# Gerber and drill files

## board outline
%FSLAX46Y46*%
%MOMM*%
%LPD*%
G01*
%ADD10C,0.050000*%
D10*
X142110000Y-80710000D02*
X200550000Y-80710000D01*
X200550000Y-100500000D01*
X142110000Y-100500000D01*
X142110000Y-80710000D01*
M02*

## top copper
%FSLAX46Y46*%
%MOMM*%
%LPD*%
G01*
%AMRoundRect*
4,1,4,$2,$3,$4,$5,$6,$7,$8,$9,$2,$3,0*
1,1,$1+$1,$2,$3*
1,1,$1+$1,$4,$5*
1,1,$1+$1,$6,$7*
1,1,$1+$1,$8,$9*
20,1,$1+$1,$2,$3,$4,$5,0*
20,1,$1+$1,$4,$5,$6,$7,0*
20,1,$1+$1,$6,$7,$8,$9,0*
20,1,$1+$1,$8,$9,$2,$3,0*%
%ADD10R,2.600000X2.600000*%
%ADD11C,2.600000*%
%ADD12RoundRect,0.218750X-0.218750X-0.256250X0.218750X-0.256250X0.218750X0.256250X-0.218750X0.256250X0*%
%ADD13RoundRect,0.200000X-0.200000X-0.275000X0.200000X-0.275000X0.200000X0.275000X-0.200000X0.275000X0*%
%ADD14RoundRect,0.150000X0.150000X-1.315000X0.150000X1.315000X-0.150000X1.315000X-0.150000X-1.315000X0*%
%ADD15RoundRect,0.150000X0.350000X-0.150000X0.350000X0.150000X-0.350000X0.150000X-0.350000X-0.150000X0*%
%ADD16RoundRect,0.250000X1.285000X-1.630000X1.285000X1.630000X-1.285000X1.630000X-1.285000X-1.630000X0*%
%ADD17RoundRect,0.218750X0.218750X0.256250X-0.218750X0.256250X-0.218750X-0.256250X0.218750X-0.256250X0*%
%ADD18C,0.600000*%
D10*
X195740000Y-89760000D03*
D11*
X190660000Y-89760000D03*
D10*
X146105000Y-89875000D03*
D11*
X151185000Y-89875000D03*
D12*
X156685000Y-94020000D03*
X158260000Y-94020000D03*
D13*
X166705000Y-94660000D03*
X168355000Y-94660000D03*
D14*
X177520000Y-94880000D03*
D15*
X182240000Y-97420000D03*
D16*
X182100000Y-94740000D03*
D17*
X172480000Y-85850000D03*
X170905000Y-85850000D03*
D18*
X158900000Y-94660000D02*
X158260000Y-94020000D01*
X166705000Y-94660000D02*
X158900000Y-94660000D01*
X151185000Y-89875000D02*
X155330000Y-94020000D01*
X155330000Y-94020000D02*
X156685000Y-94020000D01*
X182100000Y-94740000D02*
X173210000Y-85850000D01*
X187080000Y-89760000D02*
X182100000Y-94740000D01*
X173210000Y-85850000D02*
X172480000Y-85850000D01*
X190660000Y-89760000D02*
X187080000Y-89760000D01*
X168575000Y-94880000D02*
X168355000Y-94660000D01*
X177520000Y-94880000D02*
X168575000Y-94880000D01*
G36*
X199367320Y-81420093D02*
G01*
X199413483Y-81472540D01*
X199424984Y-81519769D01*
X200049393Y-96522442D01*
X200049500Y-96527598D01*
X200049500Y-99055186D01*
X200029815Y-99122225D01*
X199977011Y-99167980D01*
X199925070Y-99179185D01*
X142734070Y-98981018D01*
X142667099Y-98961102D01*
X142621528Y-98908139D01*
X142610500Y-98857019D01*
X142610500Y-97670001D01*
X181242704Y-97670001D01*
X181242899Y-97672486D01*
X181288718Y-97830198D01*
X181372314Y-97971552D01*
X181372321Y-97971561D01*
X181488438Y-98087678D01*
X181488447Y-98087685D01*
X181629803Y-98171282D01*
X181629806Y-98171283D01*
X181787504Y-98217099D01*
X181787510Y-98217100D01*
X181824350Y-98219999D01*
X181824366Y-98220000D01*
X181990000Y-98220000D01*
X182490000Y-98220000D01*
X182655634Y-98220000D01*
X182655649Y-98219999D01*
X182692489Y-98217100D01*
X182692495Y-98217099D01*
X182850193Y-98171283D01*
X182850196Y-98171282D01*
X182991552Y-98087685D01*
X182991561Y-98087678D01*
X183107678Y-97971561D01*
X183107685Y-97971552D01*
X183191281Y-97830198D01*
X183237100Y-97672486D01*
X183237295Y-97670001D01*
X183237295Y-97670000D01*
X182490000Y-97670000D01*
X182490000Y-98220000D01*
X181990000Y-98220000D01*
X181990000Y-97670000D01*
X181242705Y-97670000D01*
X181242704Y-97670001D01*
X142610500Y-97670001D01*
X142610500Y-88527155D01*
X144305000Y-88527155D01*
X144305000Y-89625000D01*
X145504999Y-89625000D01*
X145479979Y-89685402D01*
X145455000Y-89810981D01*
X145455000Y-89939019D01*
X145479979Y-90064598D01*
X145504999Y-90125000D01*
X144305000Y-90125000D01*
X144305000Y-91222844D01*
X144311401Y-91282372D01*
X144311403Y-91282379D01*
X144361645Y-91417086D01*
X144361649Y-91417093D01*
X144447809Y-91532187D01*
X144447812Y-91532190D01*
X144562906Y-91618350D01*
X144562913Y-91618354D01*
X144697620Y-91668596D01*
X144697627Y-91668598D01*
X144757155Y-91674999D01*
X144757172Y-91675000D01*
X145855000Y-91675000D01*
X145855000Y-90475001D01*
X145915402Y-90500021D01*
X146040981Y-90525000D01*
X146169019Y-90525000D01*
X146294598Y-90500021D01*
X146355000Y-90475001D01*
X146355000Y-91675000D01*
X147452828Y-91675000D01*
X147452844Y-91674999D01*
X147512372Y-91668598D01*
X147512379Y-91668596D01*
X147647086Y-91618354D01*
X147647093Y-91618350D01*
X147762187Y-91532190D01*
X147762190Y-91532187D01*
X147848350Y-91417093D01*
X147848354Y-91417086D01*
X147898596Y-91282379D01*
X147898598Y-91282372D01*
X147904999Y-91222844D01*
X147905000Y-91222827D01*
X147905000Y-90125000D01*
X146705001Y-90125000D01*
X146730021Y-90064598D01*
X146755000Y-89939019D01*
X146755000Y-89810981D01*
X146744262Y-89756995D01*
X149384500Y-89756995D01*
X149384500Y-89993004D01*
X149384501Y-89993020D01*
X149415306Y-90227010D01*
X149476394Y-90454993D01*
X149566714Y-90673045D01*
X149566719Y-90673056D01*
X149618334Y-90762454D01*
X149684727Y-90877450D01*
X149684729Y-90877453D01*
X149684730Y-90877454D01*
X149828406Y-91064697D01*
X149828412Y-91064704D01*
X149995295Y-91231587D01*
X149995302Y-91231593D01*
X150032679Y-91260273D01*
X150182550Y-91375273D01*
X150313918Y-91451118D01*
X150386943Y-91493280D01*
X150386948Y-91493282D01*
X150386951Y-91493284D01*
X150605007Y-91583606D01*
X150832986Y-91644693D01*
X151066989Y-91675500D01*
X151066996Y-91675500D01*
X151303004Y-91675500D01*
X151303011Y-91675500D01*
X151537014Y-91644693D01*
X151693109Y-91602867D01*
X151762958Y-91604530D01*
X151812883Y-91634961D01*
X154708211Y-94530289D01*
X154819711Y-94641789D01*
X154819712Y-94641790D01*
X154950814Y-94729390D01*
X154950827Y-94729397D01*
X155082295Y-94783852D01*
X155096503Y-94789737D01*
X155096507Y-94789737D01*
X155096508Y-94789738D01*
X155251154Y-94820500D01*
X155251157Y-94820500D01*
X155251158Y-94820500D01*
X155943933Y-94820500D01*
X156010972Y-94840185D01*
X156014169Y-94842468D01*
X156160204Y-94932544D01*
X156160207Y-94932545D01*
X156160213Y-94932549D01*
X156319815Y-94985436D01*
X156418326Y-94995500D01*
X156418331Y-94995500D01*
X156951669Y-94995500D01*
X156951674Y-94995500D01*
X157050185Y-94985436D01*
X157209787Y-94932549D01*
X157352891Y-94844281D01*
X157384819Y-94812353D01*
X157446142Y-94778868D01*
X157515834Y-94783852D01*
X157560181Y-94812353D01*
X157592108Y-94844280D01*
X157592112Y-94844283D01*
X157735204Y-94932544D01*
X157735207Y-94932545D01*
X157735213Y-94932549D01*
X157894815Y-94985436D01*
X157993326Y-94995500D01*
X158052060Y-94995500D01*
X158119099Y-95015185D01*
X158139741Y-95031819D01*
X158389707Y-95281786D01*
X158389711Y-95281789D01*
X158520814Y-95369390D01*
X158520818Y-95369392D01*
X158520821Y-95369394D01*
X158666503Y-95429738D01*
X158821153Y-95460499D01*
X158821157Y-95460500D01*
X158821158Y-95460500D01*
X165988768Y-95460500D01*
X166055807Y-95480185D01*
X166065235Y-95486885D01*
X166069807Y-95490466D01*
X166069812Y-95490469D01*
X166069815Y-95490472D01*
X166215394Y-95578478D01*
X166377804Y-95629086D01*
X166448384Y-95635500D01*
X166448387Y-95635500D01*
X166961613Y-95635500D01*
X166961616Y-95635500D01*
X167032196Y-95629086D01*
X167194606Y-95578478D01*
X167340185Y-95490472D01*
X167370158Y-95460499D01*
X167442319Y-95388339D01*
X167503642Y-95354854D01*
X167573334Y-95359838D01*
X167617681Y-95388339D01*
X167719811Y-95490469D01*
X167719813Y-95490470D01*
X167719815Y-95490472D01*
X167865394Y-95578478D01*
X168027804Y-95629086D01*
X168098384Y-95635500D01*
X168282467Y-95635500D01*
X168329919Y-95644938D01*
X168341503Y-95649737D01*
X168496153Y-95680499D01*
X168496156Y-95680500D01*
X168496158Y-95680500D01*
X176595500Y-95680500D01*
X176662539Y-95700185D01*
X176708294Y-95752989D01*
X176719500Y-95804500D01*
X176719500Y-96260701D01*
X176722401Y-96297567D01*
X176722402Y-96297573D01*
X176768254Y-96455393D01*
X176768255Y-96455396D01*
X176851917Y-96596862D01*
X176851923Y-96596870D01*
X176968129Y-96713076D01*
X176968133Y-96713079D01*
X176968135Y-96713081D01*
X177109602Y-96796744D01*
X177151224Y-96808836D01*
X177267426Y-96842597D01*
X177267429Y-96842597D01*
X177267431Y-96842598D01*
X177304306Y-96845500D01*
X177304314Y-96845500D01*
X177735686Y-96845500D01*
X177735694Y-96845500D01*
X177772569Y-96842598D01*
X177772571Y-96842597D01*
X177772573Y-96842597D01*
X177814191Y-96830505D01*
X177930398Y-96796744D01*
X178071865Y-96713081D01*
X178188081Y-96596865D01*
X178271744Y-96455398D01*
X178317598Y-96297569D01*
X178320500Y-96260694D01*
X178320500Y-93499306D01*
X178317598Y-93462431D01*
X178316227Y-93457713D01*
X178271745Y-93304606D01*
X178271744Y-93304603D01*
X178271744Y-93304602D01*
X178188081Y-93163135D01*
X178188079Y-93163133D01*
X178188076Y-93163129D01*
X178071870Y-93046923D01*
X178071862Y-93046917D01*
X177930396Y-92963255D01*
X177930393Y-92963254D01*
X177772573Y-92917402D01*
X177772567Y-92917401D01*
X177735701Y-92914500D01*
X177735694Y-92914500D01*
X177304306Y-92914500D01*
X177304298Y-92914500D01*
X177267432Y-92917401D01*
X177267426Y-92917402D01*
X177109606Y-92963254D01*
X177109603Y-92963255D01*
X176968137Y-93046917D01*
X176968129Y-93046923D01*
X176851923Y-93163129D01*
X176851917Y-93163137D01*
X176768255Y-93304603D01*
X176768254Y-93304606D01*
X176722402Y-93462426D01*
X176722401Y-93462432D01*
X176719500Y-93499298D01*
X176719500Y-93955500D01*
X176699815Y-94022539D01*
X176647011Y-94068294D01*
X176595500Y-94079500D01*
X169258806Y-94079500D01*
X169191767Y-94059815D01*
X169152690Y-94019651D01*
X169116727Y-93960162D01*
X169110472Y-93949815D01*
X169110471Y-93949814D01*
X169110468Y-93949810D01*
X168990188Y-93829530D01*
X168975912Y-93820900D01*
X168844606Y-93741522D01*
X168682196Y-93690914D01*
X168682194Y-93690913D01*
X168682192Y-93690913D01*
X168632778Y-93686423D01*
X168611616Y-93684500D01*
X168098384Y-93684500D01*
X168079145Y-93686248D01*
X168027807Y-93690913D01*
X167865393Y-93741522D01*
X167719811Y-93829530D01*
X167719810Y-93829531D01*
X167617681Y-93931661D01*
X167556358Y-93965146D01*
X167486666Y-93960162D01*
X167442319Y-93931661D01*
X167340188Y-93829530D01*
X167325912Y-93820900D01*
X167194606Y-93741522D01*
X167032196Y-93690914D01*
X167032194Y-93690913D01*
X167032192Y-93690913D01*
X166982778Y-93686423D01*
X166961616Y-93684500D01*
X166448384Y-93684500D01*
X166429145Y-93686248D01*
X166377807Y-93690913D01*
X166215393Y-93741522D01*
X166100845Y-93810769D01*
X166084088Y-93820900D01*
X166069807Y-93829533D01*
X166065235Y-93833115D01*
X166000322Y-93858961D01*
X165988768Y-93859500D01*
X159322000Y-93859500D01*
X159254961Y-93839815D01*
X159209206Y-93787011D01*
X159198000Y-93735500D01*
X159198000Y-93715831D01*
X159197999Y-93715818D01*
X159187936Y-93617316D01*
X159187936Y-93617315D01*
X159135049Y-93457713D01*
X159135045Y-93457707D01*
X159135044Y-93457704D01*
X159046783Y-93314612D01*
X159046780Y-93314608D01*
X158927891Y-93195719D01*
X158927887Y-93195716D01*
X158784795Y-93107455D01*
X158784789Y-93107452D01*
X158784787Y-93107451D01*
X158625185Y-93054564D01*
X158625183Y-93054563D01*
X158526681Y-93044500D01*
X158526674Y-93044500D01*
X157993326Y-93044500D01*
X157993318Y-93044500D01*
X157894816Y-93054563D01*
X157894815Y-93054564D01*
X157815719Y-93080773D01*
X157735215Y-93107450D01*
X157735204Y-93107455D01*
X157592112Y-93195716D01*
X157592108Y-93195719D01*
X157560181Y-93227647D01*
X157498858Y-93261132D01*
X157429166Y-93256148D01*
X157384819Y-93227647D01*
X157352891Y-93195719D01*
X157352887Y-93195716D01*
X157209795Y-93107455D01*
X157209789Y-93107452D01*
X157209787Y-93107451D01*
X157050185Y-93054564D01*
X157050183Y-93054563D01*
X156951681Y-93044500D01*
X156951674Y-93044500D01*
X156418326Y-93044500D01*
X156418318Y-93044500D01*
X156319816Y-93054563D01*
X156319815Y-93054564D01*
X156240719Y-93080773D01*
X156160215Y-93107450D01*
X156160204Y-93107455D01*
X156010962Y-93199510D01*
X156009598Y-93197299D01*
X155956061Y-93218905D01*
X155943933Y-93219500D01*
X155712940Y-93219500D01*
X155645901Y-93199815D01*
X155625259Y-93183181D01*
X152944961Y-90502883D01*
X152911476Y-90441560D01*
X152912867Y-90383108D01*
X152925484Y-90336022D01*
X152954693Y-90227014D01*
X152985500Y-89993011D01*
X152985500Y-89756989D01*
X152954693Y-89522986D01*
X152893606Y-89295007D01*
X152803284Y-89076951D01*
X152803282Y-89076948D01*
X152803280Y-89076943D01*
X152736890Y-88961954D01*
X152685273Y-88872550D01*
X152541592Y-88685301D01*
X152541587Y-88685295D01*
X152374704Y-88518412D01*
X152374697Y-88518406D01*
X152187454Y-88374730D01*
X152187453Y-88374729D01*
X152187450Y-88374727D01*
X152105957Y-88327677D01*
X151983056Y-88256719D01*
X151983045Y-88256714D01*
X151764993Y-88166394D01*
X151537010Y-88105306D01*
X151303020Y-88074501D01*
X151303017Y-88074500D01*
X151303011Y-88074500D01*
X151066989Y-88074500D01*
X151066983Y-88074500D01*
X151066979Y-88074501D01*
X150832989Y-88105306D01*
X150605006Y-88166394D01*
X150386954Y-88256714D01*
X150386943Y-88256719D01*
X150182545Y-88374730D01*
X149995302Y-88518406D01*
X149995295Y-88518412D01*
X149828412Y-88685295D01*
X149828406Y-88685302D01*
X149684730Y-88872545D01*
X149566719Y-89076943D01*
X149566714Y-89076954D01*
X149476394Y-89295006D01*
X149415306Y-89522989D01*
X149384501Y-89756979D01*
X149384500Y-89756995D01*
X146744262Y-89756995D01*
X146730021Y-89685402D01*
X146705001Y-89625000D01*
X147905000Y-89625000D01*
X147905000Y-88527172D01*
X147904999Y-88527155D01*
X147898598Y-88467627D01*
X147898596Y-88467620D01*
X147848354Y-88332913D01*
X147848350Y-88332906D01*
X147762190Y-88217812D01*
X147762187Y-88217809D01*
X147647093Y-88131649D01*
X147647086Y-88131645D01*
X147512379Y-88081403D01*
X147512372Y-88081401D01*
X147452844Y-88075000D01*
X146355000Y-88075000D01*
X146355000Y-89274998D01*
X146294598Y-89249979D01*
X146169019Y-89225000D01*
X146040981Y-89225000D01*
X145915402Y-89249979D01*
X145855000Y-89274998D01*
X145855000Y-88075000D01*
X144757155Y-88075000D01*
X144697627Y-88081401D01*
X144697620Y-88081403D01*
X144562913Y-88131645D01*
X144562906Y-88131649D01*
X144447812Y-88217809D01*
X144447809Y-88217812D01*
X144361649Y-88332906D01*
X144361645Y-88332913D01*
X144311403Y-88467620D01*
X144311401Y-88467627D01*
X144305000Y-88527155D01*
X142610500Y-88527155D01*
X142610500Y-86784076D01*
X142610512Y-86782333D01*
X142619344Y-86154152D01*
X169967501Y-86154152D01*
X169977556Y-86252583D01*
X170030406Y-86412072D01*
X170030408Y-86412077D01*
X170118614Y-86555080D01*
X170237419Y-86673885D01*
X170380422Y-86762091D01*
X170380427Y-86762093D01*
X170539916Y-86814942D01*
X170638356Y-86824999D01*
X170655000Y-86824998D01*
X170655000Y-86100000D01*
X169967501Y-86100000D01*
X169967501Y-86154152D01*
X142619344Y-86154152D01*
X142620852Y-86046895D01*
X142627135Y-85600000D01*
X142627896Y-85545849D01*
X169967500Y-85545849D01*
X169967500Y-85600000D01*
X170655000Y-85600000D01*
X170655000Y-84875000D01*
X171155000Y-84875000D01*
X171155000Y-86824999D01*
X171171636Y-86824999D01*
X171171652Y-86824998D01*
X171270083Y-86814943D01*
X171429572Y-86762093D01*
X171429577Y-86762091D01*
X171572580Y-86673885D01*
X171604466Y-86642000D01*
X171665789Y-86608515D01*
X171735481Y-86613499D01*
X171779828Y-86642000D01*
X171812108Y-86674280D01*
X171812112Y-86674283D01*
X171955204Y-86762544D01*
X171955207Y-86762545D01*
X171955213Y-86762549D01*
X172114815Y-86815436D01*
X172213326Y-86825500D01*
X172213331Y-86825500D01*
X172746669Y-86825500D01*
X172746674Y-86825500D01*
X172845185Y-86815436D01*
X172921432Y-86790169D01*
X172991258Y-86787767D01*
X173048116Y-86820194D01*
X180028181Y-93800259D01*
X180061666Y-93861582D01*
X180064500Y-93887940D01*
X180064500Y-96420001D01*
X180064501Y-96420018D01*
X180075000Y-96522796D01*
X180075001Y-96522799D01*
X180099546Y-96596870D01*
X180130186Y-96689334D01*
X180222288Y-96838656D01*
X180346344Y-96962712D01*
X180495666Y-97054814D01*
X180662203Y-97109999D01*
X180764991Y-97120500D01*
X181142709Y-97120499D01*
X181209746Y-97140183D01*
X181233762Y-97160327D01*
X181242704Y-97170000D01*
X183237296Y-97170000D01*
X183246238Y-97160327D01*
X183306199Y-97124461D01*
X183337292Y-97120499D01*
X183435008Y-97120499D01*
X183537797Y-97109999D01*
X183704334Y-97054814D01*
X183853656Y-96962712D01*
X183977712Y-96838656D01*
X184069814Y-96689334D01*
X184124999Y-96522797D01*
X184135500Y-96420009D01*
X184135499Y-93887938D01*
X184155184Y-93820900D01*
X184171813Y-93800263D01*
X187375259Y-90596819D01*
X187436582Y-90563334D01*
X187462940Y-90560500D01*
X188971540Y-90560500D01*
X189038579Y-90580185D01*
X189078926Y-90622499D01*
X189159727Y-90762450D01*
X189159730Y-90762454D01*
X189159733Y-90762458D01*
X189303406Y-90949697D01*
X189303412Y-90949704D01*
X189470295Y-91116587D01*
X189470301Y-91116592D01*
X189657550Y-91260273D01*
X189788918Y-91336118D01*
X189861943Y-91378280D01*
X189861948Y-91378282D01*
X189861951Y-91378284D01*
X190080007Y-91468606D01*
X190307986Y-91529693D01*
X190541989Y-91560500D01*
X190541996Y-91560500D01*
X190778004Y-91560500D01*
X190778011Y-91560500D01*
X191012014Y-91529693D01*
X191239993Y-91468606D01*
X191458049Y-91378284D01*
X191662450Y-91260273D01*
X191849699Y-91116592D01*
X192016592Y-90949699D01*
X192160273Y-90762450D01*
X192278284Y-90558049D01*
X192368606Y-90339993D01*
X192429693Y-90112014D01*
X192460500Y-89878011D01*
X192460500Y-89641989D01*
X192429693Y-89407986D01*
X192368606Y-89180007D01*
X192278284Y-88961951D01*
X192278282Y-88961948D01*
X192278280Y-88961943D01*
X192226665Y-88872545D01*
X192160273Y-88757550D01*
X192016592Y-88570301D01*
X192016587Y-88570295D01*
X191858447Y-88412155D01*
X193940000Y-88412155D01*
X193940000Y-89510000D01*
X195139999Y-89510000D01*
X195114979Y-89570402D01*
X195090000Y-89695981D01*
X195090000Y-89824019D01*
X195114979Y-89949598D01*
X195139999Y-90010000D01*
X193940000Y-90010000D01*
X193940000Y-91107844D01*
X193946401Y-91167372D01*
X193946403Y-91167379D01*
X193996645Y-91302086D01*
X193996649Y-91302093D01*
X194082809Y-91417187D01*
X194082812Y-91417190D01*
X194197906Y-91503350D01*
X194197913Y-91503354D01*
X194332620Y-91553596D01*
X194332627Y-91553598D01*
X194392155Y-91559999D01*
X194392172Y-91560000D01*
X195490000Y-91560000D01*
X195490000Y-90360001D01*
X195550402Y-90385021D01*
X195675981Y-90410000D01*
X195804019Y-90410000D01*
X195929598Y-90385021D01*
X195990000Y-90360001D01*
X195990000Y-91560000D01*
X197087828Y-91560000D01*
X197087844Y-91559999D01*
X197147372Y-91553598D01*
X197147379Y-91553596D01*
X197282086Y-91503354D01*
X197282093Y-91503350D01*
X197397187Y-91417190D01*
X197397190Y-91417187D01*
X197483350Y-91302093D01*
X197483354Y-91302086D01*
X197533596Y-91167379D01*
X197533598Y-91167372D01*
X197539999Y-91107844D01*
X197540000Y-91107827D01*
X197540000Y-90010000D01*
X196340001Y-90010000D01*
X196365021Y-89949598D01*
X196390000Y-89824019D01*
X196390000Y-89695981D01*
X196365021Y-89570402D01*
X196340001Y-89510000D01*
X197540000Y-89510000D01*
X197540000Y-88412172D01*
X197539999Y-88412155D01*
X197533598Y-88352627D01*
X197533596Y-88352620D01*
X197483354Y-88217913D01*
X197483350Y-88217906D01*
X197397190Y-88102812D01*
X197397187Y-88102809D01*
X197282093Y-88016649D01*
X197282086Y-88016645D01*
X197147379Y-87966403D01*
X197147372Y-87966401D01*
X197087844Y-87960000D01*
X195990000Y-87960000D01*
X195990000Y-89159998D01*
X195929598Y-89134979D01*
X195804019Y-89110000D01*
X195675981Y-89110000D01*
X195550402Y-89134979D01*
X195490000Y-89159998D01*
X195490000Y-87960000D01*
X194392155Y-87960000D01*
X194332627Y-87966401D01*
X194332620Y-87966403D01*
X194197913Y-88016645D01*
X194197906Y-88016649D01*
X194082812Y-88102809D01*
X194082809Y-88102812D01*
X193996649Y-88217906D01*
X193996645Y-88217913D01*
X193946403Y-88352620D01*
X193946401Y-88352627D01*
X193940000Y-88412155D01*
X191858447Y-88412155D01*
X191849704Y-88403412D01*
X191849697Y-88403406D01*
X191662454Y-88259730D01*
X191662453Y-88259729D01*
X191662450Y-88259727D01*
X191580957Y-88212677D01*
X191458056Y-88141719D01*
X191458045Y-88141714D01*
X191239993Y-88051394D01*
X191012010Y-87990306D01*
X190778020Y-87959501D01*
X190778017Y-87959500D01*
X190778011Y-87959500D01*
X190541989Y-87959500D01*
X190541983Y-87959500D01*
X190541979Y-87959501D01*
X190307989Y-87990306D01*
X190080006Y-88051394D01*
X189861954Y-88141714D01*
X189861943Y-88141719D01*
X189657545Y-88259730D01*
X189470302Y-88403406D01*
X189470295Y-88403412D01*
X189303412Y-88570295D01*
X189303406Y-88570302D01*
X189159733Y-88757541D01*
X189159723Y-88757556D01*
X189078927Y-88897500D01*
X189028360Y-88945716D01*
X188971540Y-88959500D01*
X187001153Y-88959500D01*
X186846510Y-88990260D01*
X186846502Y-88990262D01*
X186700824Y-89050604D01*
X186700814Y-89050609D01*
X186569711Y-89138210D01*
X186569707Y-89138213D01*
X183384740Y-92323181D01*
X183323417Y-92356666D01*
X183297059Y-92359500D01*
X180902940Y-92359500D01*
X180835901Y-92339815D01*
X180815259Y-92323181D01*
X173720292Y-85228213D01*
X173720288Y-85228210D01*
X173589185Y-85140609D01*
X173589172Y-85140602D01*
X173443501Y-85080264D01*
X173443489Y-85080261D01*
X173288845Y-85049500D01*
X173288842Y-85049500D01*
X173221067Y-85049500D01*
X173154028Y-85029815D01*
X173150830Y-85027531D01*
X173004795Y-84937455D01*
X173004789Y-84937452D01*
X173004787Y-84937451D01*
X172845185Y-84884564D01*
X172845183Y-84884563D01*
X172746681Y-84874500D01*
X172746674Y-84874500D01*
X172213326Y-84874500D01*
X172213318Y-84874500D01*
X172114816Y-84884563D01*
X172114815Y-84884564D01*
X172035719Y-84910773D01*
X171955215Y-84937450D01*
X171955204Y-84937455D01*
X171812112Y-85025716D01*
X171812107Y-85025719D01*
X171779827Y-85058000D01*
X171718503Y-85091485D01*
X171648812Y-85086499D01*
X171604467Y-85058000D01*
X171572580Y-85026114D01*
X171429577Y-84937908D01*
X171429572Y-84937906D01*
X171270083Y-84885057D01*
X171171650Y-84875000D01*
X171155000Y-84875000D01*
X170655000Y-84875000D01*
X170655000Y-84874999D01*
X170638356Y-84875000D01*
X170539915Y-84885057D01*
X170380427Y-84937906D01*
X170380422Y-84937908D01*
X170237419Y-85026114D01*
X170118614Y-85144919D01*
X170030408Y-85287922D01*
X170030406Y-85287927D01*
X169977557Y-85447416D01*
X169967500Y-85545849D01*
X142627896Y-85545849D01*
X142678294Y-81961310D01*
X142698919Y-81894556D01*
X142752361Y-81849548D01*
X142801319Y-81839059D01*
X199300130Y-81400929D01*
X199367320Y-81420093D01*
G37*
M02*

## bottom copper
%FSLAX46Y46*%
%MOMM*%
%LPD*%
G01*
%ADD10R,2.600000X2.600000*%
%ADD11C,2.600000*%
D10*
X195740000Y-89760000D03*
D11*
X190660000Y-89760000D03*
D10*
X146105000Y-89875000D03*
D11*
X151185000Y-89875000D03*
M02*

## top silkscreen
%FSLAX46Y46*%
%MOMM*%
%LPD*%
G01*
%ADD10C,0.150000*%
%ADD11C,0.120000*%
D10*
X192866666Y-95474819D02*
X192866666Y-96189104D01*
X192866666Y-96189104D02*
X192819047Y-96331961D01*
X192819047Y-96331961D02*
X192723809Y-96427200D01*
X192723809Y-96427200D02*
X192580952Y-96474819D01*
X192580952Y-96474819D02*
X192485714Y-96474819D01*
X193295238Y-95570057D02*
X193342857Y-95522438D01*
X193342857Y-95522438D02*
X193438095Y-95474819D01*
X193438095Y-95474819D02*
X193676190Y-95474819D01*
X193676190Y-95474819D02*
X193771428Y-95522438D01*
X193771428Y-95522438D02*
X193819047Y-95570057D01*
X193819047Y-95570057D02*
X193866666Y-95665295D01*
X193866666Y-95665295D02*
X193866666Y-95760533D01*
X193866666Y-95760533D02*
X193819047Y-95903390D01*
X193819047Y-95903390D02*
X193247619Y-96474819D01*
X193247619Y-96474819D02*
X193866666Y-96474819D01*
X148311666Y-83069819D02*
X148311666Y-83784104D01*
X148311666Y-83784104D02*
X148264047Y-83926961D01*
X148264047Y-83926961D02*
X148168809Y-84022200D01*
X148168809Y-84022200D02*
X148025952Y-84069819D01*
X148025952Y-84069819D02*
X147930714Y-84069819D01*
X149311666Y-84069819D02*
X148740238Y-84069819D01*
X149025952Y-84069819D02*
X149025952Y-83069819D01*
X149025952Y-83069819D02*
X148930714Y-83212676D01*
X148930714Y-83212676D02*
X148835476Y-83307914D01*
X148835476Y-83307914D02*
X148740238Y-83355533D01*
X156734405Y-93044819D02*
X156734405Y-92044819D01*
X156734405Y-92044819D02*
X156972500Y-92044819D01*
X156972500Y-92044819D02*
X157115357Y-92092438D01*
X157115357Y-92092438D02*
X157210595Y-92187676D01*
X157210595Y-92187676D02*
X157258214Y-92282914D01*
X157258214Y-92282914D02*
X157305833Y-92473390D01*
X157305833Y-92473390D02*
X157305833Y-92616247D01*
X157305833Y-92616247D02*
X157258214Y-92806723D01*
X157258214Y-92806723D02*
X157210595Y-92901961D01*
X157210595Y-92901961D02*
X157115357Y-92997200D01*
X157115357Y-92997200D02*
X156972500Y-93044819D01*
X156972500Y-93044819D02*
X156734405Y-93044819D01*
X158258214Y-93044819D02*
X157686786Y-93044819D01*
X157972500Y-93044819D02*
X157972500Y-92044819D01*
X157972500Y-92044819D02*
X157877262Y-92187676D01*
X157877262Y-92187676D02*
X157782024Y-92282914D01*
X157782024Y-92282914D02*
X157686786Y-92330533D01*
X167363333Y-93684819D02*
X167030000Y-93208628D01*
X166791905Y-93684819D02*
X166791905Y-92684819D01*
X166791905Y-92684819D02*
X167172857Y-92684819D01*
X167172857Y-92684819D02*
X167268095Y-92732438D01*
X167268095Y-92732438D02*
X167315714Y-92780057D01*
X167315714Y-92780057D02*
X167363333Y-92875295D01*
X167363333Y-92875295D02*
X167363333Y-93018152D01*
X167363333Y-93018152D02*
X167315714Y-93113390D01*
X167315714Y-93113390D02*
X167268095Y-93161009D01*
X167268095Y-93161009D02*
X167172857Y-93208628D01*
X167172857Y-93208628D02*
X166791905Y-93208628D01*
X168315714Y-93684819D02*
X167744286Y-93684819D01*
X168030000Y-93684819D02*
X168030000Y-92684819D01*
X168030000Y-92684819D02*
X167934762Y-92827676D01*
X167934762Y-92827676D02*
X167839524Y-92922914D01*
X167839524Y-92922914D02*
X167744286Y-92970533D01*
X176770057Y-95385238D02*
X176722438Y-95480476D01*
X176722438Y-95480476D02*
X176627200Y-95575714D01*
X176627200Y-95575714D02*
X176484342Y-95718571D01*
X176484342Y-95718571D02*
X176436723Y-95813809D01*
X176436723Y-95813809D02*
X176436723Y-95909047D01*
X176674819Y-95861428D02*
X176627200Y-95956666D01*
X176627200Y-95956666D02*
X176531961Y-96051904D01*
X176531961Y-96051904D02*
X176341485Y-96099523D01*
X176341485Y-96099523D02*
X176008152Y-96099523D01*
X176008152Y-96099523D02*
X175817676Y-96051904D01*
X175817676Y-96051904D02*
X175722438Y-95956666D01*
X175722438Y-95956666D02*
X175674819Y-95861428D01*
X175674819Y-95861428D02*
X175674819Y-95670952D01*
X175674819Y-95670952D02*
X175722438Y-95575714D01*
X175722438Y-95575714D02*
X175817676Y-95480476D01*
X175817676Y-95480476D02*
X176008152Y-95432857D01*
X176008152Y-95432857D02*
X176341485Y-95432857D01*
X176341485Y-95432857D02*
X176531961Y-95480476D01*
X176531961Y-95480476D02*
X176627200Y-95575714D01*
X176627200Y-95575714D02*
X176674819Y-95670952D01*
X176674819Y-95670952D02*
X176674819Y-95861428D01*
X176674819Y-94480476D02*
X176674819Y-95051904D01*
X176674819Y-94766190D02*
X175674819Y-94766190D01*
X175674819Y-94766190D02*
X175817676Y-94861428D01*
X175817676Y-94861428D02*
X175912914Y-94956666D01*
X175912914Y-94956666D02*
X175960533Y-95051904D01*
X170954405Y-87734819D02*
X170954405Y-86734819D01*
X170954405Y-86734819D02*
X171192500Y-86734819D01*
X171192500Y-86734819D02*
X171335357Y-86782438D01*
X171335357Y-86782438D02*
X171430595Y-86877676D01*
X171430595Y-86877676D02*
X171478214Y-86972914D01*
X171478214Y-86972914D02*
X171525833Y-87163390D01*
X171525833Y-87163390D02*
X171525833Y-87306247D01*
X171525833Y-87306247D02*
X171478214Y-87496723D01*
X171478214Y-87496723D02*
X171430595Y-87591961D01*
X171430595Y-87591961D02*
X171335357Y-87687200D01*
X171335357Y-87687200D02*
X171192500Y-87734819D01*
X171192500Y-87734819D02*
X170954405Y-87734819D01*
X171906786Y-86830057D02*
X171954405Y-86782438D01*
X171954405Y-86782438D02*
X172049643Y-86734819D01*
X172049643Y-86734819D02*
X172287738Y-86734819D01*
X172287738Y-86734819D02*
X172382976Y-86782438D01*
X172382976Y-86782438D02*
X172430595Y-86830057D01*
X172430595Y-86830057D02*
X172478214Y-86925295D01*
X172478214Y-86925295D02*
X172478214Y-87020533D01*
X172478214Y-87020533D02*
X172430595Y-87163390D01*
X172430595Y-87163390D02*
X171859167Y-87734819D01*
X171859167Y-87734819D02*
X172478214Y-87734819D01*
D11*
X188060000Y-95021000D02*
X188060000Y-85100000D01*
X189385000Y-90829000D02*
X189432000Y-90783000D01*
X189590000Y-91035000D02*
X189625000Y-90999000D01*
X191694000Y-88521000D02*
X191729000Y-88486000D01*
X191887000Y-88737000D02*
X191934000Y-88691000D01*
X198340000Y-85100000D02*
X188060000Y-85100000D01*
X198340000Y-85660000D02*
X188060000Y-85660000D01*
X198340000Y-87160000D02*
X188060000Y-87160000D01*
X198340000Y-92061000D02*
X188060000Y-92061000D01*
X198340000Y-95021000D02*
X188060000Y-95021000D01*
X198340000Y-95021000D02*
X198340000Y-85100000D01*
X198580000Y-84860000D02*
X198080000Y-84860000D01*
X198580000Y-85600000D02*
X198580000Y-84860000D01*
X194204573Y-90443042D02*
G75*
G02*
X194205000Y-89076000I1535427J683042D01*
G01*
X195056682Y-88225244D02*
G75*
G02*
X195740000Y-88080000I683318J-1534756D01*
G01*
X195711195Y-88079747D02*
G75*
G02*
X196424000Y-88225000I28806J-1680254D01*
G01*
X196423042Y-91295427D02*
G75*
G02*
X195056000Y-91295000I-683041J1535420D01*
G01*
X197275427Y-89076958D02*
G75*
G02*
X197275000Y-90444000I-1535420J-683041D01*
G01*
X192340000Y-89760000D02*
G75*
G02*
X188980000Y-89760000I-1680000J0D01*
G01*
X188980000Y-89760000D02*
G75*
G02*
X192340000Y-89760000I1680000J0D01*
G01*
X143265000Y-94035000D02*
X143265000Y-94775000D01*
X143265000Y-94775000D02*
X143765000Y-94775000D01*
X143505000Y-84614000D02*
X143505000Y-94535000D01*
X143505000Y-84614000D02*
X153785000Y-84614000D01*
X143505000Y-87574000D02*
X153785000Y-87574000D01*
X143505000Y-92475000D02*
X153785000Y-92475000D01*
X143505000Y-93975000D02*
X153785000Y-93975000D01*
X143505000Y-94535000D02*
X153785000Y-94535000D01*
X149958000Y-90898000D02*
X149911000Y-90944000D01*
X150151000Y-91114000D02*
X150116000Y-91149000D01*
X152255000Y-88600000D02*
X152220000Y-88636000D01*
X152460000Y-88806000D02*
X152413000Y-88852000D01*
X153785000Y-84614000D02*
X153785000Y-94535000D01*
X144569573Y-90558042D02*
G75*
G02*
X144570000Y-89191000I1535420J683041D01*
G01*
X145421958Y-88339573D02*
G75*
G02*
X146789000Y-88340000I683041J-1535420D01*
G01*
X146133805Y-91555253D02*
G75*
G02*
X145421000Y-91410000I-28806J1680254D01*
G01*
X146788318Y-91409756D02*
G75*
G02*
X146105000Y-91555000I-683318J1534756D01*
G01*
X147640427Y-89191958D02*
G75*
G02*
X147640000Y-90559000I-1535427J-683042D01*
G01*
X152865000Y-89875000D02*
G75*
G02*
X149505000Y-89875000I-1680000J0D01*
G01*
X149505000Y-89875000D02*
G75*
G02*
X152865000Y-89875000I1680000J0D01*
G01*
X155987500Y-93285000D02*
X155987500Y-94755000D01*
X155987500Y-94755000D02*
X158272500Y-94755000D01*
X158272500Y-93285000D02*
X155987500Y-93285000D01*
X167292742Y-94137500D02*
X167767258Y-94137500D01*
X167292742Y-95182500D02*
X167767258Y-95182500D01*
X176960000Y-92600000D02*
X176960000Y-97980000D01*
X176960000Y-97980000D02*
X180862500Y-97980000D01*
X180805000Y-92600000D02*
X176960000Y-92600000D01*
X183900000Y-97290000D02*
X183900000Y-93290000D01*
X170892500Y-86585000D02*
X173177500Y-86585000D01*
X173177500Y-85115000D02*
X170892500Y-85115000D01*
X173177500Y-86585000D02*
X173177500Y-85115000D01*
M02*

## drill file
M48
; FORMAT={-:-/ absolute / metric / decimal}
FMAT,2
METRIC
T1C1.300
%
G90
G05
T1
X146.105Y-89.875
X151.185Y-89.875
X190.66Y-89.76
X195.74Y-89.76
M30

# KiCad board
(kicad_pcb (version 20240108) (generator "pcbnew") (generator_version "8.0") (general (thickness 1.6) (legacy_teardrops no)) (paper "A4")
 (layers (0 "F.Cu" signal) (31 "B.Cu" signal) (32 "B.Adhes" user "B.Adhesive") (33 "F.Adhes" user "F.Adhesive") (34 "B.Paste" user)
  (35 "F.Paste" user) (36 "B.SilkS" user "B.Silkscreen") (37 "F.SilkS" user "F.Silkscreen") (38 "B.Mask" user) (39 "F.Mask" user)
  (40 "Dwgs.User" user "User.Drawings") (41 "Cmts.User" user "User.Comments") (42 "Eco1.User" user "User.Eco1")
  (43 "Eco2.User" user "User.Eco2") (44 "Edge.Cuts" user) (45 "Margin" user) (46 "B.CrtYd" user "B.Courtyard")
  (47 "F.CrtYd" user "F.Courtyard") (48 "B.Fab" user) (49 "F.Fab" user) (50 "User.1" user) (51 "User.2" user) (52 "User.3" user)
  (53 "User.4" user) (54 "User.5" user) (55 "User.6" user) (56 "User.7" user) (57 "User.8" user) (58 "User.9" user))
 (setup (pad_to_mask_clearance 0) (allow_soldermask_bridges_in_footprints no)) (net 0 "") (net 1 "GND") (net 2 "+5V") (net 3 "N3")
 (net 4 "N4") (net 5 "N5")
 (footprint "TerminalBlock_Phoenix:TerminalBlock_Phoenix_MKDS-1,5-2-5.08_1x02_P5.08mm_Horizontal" (layer "F.Cu") (at 195.74 89.76 180)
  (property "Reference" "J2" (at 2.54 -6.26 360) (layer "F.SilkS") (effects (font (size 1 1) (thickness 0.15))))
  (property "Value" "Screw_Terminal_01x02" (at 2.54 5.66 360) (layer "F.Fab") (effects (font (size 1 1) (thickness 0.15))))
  (fp_line (start 7.68 -5.261) (end 7.68 4.66) (stroke (width 0.12) (type solid)) (layer "F.SilkS"))
  (fp_line (start 6.355 -1.069) (end 6.308 -1.023) (stroke (width 0.12) (type solid)) (layer "F.SilkS"))
  (fp_line (start 6.15 -1.275) (end 6.115 -1.239) (stroke (width 0.12) (type solid)) (layer "F.SilkS"))
  (fp_line (start 4.046 1.239) (end 4.011 1.274) (stroke (width 0.12) (type solid)) (layer "F.SilkS"))
  (fp_line (start 3.853 1.023) (end 3.806 1.069) (stroke (width 0.12) (type solid)) (layer "F.SilkS"))
  (fp_line (start -2.6 4.66) (end 7.68 4.66) (stroke (width 0.12) (type solid)) (layer "F.SilkS"))
  (fp_line (start -2.6 4.1) (end 7.68 4.1) (stroke (width 0.12) (type solid)) (layer "F.SilkS"))
  (fp_line (start -2.6 2.6) (end 7.68 2.6) (stroke (width 0.12) (type solid)) (layer "F.SilkS"))
  (fp_line (start -2.6 -2.301) (end 7.68 -2.301) (stroke (width 0.12) (type solid)) (layer "F.SilkS"))
  (fp_line (start -2.6 -5.261) (end 7.68 -5.261) (stroke (width 0.12) (type solid)) (layer "F.SilkS"))
  (fp_line (start -2.6 -5.261) (end -2.6 4.66) (stroke (width 0.12) (type solid)) (layer "F.SilkS"))
  (fp_line (start -2.84 4.9) (end -2.34 4.9) (stroke (width 0.12) (type solid)) (layer "F.SilkS"))
  (fp_line (start -2.84 4.16) (end -2.84 4.9) (stroke (width 0.12) (type solid)) (layer "F.SilkS"))
  (fp_arc (start 1.535427 -0.683042) (mid 1.680501 0.000524) (end 1.535 0.684) (stroke (width 0.12) (type solid)) (layer "F.SilkS"))
  (fp_arc (start 0.683318 1.534756) (mid 0.349292 1.643288) (end 0 1.68) (stroke (width 0.12) (type solid)) (layer "F.SilkS"))
  (fp_arc (start 0.028805 1.680253) (mid -0.335551 1.646659) (end -0.684 1.535) (stroke (width 0.12) (type solid)) (layer "F.SilkS"))
  (fp_arc (start -0.683042 -1.535427) (mid 0.000524 -1.680501) (end 0.684 -1.535) (stroke (width 0.12) (type solid)) (layer "F.SilkS"))
  (fp_arc (start -1.535427 0.683042) (mid -1.680501 -0.000524) (end -1.535 -0.684) (stroke (width 0.12) (type solid)) (layer "F.SilkS"))
  (fp_circle (center 5.08 0) (end 6.76 0) (stroke (width 0.12) (type solid)) (fill none) (layer "F.SilkS"))
  (pad "1" thru_hole rect (at 0 0 180) (size 2.6 2.6) (drill 1.3) (layers "*.Cu" "*.Mask") (remove_unused_layers no) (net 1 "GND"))
  (pad "2" thru_hole circle (at 5.08 0 180) (size 2.6 2.6) (drill 1.3) (layers "*.Cu" "*.Mask") (remove_unused_layers no) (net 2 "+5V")))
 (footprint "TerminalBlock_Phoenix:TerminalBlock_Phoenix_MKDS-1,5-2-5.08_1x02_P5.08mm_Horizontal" (layer "F.Cu") (at 146.105 89.875)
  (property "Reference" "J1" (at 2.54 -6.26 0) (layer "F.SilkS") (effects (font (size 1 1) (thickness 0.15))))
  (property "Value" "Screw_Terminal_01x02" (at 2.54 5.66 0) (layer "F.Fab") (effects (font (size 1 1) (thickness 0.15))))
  (fp_line (start -2.84 4.16) (end -2.84 4.9) (stroke (width 0.12) (type solid)) (layer "F.SilkS"))
  (fp_line (start -2.84 4.9) (end -2.34 4.9) (stroke (width 0.12) (type solid)) (layer "F.SilkS"))
  (fp_line (start -2.6 -5.261) (end -2.6 4.66) (stroke (width 0.12) (type solid)) (layer "F.SilkS"))
  (fp_line (start -2.6 -5.261) (end 7.68 -5.261) (stroke (width 0.12) (type solid)) (layer "F.SilkS"))
  (fp_line (start -2.6 -2.301) (end 7.68 -2.301) (stroke (width 0.12) (type solid)) (layer "F.SilkS"))
  (fp_line (start -2.6 2.6) (end 7.68 2.6) (stroke (width 0.12) (type solid)) (layer "F.SilkS"))
  (fp_line (start -2.6 4.1) (end 7.68 4.1) (stroke (width 0.12) (type solid)) (layer "F.SilkS"))
  (fp_line (start -2.6 4.66) (end 7.68 4.66) (stroke (width 0.12) (type solid)) (layer "F.SilkS"))
  (fp_line (start 3.853 1.023) (end 3.806 1.069) (stroke (width 0.12) (type solid)) (layer "F.SilkS"))
  (fp_line (start 4.046 1.239) (end 4.011 1.274) (stroke (width 0.12) (type solid)) (layer "F.SilkS"))
  (fp_line (start 6.15 -1.275) (end 6.115 -1.239) (stroke (width 0.12) (type solid)) (layer "F.SilkS"))
  (fp_line (start 6.355 -1.069) (end 6.308 -1.023) (stroke (width 0.12) (type solid)) (layer "F.SilkS"))
  (fp_line (start 7.68 -5.261) (end 7.68 4.66) (stroke (width 0.12) (type solid)) (layer "F.SilkS"))
  (fp_arc (start -1.535427 0.683042) (mid -1.680501 -0.000524) (end -1.535 -0.684) (stroke (width 0.12) (type solid)) (layer "F.SilkS"))
  (fp_arc (start -0.683042 -1.535427) (mid 0.000524 -1.680501) (end 0.684 -1.535) (stroke (width 0.12) (type solid)) (layer "F.SilkS"))
  (fp_arc (start 0.028805 1.680253) (mid -0.335551 1.646659) (end -0.684 1.535) (stroke (width 0.12) (type solid)) (layer "F.SilkS"))
  (fp_arc (start 0.683318 1.534756) (mid 0.349292 1.643288) (end 0 1.68) (stroke (width 0.12) (type solid)) (layer "F.SilkS"))
  (fp_arc (start 1.535427 -0.683042) (mid 1.680501 0.000524) (end 1.535 0.684) (stroke (width 0.12) (type solid)) (layer "F.SilkS"))
  (fp_circle (center 5.08 0) (end 6.76 0) (stroke (width 0.12) (type solid)) (fill none) (layer "F.SilkS"))
  (pad "1" thru_hole rect (at 0 0) (size 2.6 2.6) (drill 1.3) (layers "*.Cu" "*.Mask") (remove_unused_layers no) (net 1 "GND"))
  (pad "2" thru_hole circle (at 5.08 0) (size 2.6 2.6) (drill 1.3) (layers "*.Cu" "*.Mask") (remove_unused_layers no) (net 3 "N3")))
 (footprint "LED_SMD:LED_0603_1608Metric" (layer "F.Cu") (at 157.4725 94.02)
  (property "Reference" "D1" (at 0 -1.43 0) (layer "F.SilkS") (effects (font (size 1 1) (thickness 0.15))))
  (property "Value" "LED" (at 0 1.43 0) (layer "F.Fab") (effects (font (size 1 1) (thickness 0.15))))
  (fp_line (start -1.485 -0.735) (end -1.485 0.735) (stroke (width 0.12) (type solid)) (layer "F.SilkS"))
  (fp_line (start -1.485 0.735) (end 0.8 0.735) (stroke (width 0.12) (type solid)) (layer "F.SilkS"))
  (fp_line (start 0.8 -0.735) (end -1.485 -0.735) (stroke (width 0.12) (type solid)) (layer "F.SilkS"))
  (pad "1" smd roundrect (at -0.7875 0) (size 0.875 0.95) (layers "F.Cu" "F.Paste" "F.Mask") (roundrect_rratio 0.25) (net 3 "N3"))
  (pad "2" smd roundrect (at 0.7875 0) (size 0.875 0.95) (layers "F.Cu" "F.Paste" "F.Mask") (roundrect_rratio 0.25) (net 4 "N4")))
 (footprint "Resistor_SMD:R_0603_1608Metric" (layer "F.Cu") (at 167.53 94.66)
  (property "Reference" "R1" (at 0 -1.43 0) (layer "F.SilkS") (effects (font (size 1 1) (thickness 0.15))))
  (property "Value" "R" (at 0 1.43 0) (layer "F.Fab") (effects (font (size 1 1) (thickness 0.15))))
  (fp_line (start -0.237258 -0.5225) (end 0.237258 -0.5225) (stroke (width 0.12) (type solid)) (layer "F.SilkS"))
  (fp_line (start -0.237258 0.5225) (end 0.237258 0.5225) (stroke (width 0.12) (type solid)) (layer "F.SilkS"))
  (pad "1" smd roundrect (at -0.825 0) (size 0.8 0.95) (layers "F.Cu" "F.Paste" "F.Mask") (roundrect_rratio 0.25) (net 4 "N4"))
  (pad "2" smd roundrect (at 0.825 0) (size 0.8 0.95) (layers "F.Cu" "F.Paste" "F.Mask") (roundrect_rratio 0.25) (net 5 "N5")))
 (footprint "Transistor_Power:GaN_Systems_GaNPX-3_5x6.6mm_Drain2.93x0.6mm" (layer "F.Cu") (at 180.43 95.29 90)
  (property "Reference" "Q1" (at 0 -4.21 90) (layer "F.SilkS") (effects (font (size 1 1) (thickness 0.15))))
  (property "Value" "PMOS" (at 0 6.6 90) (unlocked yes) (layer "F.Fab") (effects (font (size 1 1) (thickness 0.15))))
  (fp_line (start 2.69 -3.47) (end -2.69 -3.47) (stroke (width 0.12) (type default)) (layer "F.SilkS"))
  (fp_line (start -2.69 -3.47) (end -2.69 0.4325) (stroke (width 0.12) (type default)) (layer "F.SilkS"))
  (fp_line (start 2.69 0.375) (end 2.69 -3.47) (stroke (width 0.12) (type default)) (layer "F.SilkS"))
  (fp_line (start -2 3.47) (end 2 3.47) (stroke (width 0.12) (type default)) (layer "F.SilkS"))
  (pad "" smd roundrect (at -0.34 0.9525 90) (size 1.58 1.235) (layers "F.Paste") (roundrect_rratio 0.2024291498))
  (pad "" smd roundrect (at -0.34 2.3875 90) (size 1.58 1.235) (layers "F.Paste") (roundrect_rratio 0.2024291498))
  (pad "" smd roundrect (at 1.44 0.9525 90) (size 1.58 1.235) (layers "F.Paste") (roundrect_rratio 0.2024291498))
  (pad "" smd roundrect (at 1.44 2.3875 90) (size 1.58 1.235) (layers "F.Paste") (roundrect_rratio 0.2024291498))
  (pad "1" smd roundrect (at 0.41 -2.91 90) (size 2.93 0.6) (layers "F.Cu" "F.Paste" "F.Mask") (roundrect_rratio 0.25) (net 5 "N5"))
  (pad "2" smd roundrect (at -2.13 1.81 90) (size 0.6 1) (layers "F.Cu" "F.Paste" "F.Mask") (roundrect_rratio 0.25) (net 1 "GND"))
  (pad "3" smd roundrect (at 0.55 1.67 90) (size 3.76 3.07) (layers "F.Cu" "F.Mask") (roundrect_rratio 0.08143322476) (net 2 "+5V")))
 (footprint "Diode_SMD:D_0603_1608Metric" (layer "F.Cu") (at 171.6925 85.85 180)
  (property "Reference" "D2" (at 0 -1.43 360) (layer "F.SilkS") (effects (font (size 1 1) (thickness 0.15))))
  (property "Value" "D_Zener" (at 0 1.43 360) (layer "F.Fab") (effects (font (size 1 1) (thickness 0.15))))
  (fp_line (start 0.8 -0.735) (end -1.485 -0.735) (stroke (width 0.12) (type solid)) (layer "F.SilkS"))
  (fp_line (start -1.485 0.735) (end 0.8 0.735) (stroke (width 0.12) (type solid)) (layer "F.SilkS"))
  (fp_line (start -1.485 -0.735) (end -1.485 0.735) (stroke (width 0.12) (type solid)) (layer "F.SilkS"))
  (pad "1" smd roundrect (at -0.7875 0 180) (size 0.875 0.95) (layers "F.Cu" "F.Paste" "F.Mask") (roundrect_rratio 0.25) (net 2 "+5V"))
  (pad "2" smd roundrect (at 0.7875 0 180) (size 0.875 0.95) (layers "F.Cu" "F.Paste" "F.Mask") (roundrect_rratio 0.25) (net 1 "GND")))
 (gr_rect (start 142.11 80.71) (end 200.55 100.5) (stroke (width 0.05) (type default)) (fill none) (layer "Edge.Cuts"))
 (segment (start 158.9 94.66) (end 158.26 94.02) (width 0.6) (layer "F.Cu") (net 4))
 (segment (start 166.705 94.66) (end 158.9 94.66) (width 0.6) (layer "F.Cu") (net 4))
 (segment (start 151.185 89.875) (end 155.33 94.02) (width 0.6) (layer "F.Cu") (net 3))
 (segment (start 155.33 94.02) (end 156.685 94.02) (width 0.6) (layer "F.Cu") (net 3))
 (segment (start 182.1 94.74) (end 173.21 85.85) (width 0.6) (layer "F.Cu") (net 2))
 (segment (start 187.08 89.76) (end 182.1 94.74) (width 0.6) (layer "F.Cu") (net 2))
 (segment (start 173.21 85.85) (end 172.48 85.85) (width 0.6) (layer "F.Cu") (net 2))
 (segment (start 190.66 89.76) (end 187.08 89.76) (width 0.6) (layer "F.Cu") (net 2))
 (segment (start 168.575 94.88) (end 168.355 94.66) (width 0.6) (layer "F.Cu") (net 5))
 (segment (start 177.52 94.88) (end 168.575 94.88) (width 0.6) (layer "F.Cu") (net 5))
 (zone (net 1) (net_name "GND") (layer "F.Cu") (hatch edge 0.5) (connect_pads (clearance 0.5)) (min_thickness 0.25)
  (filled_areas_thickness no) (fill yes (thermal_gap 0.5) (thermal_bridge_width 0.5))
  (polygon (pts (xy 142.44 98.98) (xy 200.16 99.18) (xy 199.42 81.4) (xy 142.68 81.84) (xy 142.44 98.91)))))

